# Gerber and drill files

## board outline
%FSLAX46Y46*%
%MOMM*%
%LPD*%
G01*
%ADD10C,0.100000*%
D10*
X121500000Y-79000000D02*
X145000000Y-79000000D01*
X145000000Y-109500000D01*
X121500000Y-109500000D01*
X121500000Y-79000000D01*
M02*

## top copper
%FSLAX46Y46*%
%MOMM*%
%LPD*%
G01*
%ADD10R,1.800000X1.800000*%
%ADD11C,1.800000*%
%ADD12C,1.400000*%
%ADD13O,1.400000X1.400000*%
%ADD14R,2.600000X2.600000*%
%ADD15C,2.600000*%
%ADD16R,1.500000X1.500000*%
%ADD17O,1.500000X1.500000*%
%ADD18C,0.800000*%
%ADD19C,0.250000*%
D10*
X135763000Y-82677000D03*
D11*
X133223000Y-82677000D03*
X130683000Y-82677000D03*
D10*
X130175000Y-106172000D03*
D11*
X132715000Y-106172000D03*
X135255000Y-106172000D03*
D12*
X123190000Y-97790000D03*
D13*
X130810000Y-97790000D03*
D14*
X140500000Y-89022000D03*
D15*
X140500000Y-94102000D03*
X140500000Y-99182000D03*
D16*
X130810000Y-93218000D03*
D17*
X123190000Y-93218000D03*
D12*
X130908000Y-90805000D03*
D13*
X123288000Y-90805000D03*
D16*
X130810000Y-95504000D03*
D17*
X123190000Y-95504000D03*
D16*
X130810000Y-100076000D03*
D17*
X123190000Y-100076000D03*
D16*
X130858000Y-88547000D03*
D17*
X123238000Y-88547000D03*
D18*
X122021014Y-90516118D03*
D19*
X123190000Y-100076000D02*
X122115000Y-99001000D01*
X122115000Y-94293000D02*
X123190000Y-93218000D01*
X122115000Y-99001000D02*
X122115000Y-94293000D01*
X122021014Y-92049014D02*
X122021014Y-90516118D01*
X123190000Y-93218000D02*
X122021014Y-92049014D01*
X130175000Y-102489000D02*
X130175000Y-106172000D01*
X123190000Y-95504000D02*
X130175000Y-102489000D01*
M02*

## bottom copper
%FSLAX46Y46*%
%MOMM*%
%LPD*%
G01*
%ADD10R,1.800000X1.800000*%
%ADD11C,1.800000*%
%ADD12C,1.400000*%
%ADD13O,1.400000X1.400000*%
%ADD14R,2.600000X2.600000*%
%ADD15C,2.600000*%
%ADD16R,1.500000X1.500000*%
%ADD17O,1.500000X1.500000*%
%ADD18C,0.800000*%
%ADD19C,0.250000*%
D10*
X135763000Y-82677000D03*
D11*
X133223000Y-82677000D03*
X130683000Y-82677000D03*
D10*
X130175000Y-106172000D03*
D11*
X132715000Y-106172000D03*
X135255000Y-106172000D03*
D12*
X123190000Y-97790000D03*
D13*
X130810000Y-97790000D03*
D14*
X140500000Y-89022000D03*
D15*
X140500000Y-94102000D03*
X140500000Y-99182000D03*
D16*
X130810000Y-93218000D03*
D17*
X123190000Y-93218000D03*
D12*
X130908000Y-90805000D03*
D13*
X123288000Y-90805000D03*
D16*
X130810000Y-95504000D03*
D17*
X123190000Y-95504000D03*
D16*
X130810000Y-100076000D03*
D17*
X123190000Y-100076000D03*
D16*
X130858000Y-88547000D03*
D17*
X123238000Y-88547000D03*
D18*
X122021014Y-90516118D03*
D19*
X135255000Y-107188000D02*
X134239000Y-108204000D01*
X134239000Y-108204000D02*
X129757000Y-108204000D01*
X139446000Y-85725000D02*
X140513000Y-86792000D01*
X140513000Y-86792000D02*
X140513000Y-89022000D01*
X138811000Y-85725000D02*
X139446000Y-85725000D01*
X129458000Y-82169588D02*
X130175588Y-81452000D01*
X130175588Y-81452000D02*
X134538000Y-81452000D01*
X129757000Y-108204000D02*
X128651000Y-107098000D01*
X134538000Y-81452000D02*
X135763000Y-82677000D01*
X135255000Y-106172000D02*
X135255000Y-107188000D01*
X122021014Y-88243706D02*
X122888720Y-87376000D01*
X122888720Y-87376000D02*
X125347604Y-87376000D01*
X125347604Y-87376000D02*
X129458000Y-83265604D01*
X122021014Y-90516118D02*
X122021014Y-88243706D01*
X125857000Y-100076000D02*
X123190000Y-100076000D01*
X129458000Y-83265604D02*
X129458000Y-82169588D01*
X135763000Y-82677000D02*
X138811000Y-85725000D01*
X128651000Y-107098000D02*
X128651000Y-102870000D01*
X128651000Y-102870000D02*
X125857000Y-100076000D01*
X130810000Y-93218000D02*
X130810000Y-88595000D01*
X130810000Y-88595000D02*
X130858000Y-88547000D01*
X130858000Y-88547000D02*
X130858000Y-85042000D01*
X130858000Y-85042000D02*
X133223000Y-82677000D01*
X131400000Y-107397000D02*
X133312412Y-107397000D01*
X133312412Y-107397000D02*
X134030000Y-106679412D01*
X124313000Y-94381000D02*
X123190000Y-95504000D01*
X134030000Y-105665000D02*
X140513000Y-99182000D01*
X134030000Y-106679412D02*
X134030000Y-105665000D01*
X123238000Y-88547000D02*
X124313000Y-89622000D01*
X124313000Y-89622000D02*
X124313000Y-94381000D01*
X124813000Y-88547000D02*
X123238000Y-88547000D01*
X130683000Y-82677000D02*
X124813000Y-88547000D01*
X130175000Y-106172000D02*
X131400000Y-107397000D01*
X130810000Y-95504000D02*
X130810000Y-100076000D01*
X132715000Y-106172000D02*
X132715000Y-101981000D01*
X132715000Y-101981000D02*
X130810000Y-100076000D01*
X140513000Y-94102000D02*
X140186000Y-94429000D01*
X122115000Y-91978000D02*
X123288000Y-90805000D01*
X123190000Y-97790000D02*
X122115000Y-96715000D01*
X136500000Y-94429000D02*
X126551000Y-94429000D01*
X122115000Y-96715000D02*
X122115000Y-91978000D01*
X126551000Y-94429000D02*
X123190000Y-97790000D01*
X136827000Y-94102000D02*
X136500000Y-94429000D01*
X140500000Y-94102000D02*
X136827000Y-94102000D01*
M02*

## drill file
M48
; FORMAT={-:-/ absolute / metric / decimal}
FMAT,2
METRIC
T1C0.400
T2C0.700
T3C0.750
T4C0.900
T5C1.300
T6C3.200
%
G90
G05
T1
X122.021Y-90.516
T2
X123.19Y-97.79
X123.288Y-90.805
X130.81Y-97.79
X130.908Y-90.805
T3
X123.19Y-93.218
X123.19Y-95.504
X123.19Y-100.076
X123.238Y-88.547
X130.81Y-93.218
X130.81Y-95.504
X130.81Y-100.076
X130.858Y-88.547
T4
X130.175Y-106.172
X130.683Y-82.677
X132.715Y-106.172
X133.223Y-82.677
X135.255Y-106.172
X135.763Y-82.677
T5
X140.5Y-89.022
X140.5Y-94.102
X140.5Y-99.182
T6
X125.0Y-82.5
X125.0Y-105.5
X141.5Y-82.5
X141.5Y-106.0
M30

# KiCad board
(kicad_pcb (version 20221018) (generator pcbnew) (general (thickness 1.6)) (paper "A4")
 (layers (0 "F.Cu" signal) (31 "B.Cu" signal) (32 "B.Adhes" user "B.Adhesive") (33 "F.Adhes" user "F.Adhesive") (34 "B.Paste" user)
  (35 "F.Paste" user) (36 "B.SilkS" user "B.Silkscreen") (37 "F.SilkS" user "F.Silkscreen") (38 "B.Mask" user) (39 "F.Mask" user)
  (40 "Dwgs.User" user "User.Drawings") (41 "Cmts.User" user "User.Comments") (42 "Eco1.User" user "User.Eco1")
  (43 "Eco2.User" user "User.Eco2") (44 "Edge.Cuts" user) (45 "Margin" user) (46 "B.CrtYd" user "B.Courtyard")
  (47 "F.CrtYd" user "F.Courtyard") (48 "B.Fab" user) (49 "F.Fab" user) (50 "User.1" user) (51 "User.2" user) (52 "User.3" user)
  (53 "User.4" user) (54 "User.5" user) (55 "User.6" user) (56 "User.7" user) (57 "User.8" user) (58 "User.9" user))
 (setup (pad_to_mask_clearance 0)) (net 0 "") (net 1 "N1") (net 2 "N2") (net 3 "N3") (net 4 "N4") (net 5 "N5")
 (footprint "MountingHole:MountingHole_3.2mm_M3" (layer "F.Cu") (at 141.5 82.5)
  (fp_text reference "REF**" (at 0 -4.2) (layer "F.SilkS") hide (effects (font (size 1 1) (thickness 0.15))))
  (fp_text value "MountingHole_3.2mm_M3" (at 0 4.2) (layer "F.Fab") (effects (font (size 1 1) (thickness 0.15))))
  (pad "" np_thru_hole circle (at 0 0) (size 3.2 3.2) (drill 3.2) (layers "*.Cu" "*.Mask")))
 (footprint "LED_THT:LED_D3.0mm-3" (layer "F.Cu") (at 135.763 82.677 180)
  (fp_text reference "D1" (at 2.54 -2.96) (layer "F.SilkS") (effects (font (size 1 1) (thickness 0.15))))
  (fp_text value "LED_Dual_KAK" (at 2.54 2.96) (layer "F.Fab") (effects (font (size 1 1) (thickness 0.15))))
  (pad "1" thru_hole rect (at 0 0 180) (size 1.8 1.8) (drill 0.9) (layers "*.Cu" "*.Mask") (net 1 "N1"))
  (pad "2" thru_hole circle (at 2.54 0 180) (size 1.8 1.8) (drill 0.9) (layers "*.Cu" "*.Mask") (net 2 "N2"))
  (pad "3" thru_hole circle (at 5.08 0 180) (size 1.8 1.8) (drill 0.9) (layers "*.Cu" "*.Mask") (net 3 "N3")))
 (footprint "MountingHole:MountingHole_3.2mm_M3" (layer "F.Cu") (at 125 105.5)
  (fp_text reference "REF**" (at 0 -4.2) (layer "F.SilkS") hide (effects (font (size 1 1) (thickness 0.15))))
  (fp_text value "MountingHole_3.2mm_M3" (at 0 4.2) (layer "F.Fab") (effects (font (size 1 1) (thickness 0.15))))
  (pad "" np_thru_hole circle (at 0 0) (size 3.2 3.2) (drill 3.2) (layers "F&B.Cu" "*.Mask")))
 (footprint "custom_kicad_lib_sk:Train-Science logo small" (layer "F.Cu") (at 138.5 96.5 90)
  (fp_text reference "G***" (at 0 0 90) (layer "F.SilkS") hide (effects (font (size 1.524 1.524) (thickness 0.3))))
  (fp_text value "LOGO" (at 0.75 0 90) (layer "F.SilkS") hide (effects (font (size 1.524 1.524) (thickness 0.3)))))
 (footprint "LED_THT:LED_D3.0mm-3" (layer "F.Cu") (at 130.175 106.172)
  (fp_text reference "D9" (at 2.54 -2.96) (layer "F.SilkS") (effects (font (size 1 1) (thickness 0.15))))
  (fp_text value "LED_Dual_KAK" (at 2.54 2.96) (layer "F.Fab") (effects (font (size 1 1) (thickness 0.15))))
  (pad "1" thru_hole rect (at 0 0) (size 1.8 1.8) (drill 0.9) (layers "*.Cu" "*.Mask") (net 3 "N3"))
  (pad "2" thru_hole circle (at 2.54 0) (size 1.8 1.8) (drill 0.9) (layers "*.Cu" "*.Mask") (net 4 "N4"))
  (pad "3" thru_hole circle (at 5.08 0) (size 1.8 1.8) (drill 0.9) (layers "*.Cu" "*.Mask") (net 1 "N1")))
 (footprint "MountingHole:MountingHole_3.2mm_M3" (layer "F.Cu") (at 125 82.5)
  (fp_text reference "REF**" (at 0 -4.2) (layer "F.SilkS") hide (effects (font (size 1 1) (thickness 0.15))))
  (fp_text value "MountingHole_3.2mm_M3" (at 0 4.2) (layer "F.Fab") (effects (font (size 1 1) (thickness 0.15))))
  (pad "" np_thru_hole circle (at 0 0) (size 3.2 3.2) (drill 3.2) (layers "F&B.Cu" "*.Mask")))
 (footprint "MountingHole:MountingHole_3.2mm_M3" (layer "F.Cu") (at 141.5 106)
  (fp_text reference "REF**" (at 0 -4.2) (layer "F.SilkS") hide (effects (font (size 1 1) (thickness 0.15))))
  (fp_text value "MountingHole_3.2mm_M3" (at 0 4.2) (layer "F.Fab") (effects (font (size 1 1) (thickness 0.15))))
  (pad "" np_thru_hole circle (at 0 0) (size 3.2 3.2) (drill 3.2) (layers "F&B.Cu" "*.Mask")))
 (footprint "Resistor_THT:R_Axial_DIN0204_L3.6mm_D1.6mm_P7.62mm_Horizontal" (layer "B.Cu") (at 123.19 97.79)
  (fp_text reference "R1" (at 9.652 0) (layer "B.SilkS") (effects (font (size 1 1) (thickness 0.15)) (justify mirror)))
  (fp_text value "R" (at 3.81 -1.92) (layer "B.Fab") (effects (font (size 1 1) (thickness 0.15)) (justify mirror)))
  (pad "1" thru_hole circle (at 0 0) (size 1.4 1.4) (drill 0.7) (layers "*.Cu" "*.Mask") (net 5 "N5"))
  (pad "2" thru_hole oval (at 7.62 0) (size 1.4 1.4) (drill 0.7) (layers "*.Cu" "*.Mask") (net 4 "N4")))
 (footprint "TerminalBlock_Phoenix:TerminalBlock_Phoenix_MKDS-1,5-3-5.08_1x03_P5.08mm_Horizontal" (layer "B.Cu") (at 140.5 89.022 -90)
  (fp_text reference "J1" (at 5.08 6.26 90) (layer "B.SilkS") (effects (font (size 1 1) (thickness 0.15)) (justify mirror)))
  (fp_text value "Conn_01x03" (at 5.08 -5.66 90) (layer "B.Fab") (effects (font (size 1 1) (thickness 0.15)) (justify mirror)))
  (pad "1" thru_hole rect (at 0 0 270) (size 2.6 2.6) (drill 1.3) (layers "*.Cu" "*.Mask") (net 1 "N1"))
  (pad "2" thru_hole circle (at 5.08 0 270) (size 2.6 2.6) (drill 1.3) (layers "*.Cu" "*.Mask") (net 5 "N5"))
  (pad "3" thru_hole circle (at 10.16 0 270) (size 2.6 2.6) (drill 1.3) (layers "*.Cu" "*.Mask") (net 3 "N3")))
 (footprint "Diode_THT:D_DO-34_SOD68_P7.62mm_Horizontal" (layer "B.Cu") (at 130.81 93.218 180)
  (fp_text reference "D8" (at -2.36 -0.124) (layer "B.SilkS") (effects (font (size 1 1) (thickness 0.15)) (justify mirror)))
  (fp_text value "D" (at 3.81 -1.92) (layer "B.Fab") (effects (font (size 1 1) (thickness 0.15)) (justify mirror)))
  (pad "1" thru_hole rect (at 0 0 180) (size 1.5 1.5) (drill 0.75) (layers "*.Cu" "*.Mask") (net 2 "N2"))
  (pad "2" thru_hole oval (at 7.62 0 180) (size 1.5 1.5) (drill 0.75) (layers "*.Cu" "*.Mask") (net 1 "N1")))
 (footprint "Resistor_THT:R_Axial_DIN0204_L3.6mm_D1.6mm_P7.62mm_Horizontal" (layer "B.Cu") (at 130.908 90.805 180)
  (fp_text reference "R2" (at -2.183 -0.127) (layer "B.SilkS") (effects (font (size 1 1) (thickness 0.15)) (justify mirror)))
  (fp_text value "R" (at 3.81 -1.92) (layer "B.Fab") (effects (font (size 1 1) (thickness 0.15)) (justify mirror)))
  (pad "1" thru_hole circle (at 0 0 180) (size 1.4 1.4) (drill 0.7) (layers "*.Cu" "*.Mask") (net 2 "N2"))
  (pad "2" thru_hole oval (at 7.62 0 180) (size 1.4 1.4) (drill 0.7) (layers "*.Cu" "*.Mask") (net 5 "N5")))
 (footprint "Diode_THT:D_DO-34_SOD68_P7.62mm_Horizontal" (layer "B.Cu") (at 130.81 95.504 180)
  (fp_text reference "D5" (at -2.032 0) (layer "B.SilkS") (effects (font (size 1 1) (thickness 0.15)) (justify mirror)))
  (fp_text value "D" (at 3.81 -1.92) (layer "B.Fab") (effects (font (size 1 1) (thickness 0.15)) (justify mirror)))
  (pad "1" thru_hole rect (at 0 0 180) (size 1.5 1.5) (drill 0.75) (layers "*.Cu" "*.Mask") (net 4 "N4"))
  (pad "2" thru_hole oval (at 7.62 0 180) (size 1.5 1.5) (drill 0.75) (layers "*.Cu" "*.Mask") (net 3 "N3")))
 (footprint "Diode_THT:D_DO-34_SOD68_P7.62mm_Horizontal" (layer "B.Cu") (at 130.81 100.076 180)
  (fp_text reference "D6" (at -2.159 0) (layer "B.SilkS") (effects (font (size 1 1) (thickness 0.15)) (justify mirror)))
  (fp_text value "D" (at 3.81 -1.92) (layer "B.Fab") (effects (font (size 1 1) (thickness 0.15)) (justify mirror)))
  (pad "1" thru_hole rect (at 0 0 180) (size 1.5 1.5) (drill 0.75) (layers "*.Cu" "*.Mask") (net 4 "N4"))
  (pad "2" thru_hole oval (at 7.62 0 180) (size 1.5 1.5) (drill 0.75) (layers "*.Cu" "*.Mask") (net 1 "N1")))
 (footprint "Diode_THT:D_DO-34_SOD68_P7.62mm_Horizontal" (layer "B.Cu") (at 130.858 88.547 180)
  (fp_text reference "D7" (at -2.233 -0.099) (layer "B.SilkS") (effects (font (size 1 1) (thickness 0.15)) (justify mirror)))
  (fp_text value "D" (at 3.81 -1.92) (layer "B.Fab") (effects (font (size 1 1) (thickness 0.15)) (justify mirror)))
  (pad "1" thru_hole rect (at 0 0 180) (size 1.5 1.5) (drill 0.75) (layers "*.Cu" "*.Mask") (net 2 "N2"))
  (pad "2" thru_hole oval (at 7.62 0 180) (size 1.5 1.5) (drill 0.75) (layers "*.Cu" "*.Mask") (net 3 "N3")))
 (gr_rect (start 121.5 79) (end 145 109.5) (stroke (width 0.1) (type default)) (fill none) (layer "Edge.Cuts"))
 (segment (start 123.19 100.076) (end 122.115 99.001) (width 0.25) (layer "F.Cu") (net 1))
 (segment (start 122.115 94.293) (end 123.19 93.218) (width 0.25) (layer "F.Cu") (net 1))
 (segment (start 122.115 99.001) (end 122.115 94.293) (width 0.25) (layer "F.Cu") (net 1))
 (segment (start 122.021014 92.049014) (end 122.021014 90.516118) (width 0.25) (layer "F.Cu") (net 1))
 (segment (start 123.19 93.218) (end 122.021014 92.049014) (width 0.25) (layer "F.Cu") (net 1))
 (via (at 122.021014 90.516118) (size 0.8) (drill 0.4) (layers "F.Cu" "B.Cu") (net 1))
 (segment (start 135.255 107.188) (end 134.239 108.204) (width 0.25) (layer "B.Cu") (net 1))
 (segment (start 134.239 108.204) (end 129.757 108.204) (width 0.25) (layer "B.Cu") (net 1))
 (segment (start 139.446 85.725) (end 140.513 86.792) (width 0.25) (layer "B.Cu") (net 1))
 (segment (start 140.513 86.792) (end 140.513 89.022) (width 0.25) (layer "B.Cu") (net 1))
 (segment (start 138.811 85.725) (end 139.446 85.725) (width 0.25) (layer "B.Cu") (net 1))
 (segment (start 129.458 82.169588) (end 130.175588 81.452) (width 0.25) (layer "B.Cu") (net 1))
 (segment (start 130.175588 81.452) (end 134.538 81.452) (width 0.25) (layer "B.Cu") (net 1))
 (segment (start 129.757 108.204) (end 128.651 107.098) (width 0.25) (layer "B.Cu") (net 1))
 (segment (start 134.538 81.452) (end 135.763 82.677) (width 0.25) (layer "B.Cu") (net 1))
 (segment (start 135.255 106.172) (end 135.255 107.188) (width 0.25) (layer "B.Cu") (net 1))
 (segment (start 122.021014 88.243706) (end 122.88872 87.376) (width 0.25) (layer "B.Cu") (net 1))
 (segment (start 122.88872 87.376) (end 125.347604 87.376) (width 0.25) (layer "B.Cu") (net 1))
 (segment (start 125.347604 87.376) (end 129.458 83.265604) (width 0.25) (layer "B.Cu") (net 1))
 (segment (start 122.021014 90.516118) (end 122.021014 88.243706) (width 0.25) (layer "B.Cu") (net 1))
 (segment (start 125.857 100.076) (end 123.19 100.076) (width 0.25) (layer "B.Cu") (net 1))
 (segment (start 129.458 83.265604) (end 129.458 82.169588) (width 0.25) (layer "B.Cu") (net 1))
 (segment (start 135.763 82.677) (end 138.811 85.725) (width 0.25) (layer "B.Cu") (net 1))
 (segment (start 128.651 107.098) (end 128.651 102.87) (width 0.25) (layer "B.Cu") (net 1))
 (segment (start 128.651 102.87) (end 125.857 100.076) (width 0.25) (layer "B.Cu") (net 1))
 (segment (start 130.81 93.218) (end 130.81 88.595) (width 0.25) (layer "B.Cu") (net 2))
 (segment (start 130.81 88.595) (end 130.858 88.547) (width 0.25) (layer "B.Cu") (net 2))
 (segment (start 130.858 88.547) (end 130.858 85.042) (width 0.25) (layer "B.Cu") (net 2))
 (segment (start 130.858 85.042) (end 133.223 82.677) (width 0.25) (layer "B.Cu") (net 2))
 (segment (start 130.175 102.489) (end 130.175 106.172) (width 0.25) (layer "F.Cu") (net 3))
 (segment (start 123.19 95.504) (end 130.175 102.489) (width 0.25) (layer "F.Cu") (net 3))
 (segment (start 131.4 107.397) (end 133.312412 107.397) (width 0.25) (layer "B.Cu") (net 3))
 (segment (start 133.312412 107.397) (end 134.03 106.679412) (width 0.25) (layer "B.Cu") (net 3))
 (segment (start 124.313 94.381) (end 123.19 95.504) (width 0.25) (layer "B.Cu") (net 3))
 (segment (start 134.03 105.665) (end 140.513 99.182) (width 0.25) (layer "B.Cu") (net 3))
 (segment (start 134.03 106.679412) (end 134.03 105.665) (width 0.25) (layer "B.Cu") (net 3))
 (segment (start 123.238 88.547) (end 124.313 89.622) (width 0.25) (layer "B.Cu") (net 3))
 (segment (start 124.313 89.622) (end 124.313 94.381) (width 0.25) (layer "B.Cu") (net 3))
 (segment (start 124.813 88.547) (end 123.238 88.547) (width 0.25) (layer "B.Cu") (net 3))
 (segment (start 130.683 82.677) (end 124.813 88.547) (width 0.25) (layer "B.Cu") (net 3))
 (segment (start 130.175 106.172) (end 131.4 107.397) (width 0.25) (layer "B.Cu") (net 3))
 (segment (start 130.81 95.504) (end 130.81 100.076) (width 0.25) (layer "B.Cu") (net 4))
 (segment (start 132.715 106.172) (end 132.715 101.981) (width 0.25) (layer "B.Cu") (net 4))
 (segment (start 132.715 101.981) (end 130.81 100.076) (width 0.25) (layer "B.Cu") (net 4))
 (segment (start 140.513 94.102) (end 140.186 94.429) (width 0.25) (layer "B.Cu") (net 5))
 (segment (start 122.115 91.978) (end 123.288 90.805) (width 0.25) (layer "B.Cu") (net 5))
 (segment (start 123.19 97.79) (end 122.115 96.715) (width 0.25) (layer "B.Cu") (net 5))
 (segment (start 136.5 94.429) (end 126.551 94.429) (width 0.25) (layer "B.Cu") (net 5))
 (segment (start 122.115 96.715) (end 122.115 91.978) (width 0.25) (layer "B.Cu") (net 5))
 (segment (start 126.551 94.429) (end 123.19 97.79) (width 0.25) (layer "B.Cu") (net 5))
 (segment (start 136.827 94.102) (end 136.5 94.429) (width 0.25) (layer "B.Cu") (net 5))
 (segment (start 140.5 94.102) (end 136.827 94.102) (width 0.25) (layer "B.Cu") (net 5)))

